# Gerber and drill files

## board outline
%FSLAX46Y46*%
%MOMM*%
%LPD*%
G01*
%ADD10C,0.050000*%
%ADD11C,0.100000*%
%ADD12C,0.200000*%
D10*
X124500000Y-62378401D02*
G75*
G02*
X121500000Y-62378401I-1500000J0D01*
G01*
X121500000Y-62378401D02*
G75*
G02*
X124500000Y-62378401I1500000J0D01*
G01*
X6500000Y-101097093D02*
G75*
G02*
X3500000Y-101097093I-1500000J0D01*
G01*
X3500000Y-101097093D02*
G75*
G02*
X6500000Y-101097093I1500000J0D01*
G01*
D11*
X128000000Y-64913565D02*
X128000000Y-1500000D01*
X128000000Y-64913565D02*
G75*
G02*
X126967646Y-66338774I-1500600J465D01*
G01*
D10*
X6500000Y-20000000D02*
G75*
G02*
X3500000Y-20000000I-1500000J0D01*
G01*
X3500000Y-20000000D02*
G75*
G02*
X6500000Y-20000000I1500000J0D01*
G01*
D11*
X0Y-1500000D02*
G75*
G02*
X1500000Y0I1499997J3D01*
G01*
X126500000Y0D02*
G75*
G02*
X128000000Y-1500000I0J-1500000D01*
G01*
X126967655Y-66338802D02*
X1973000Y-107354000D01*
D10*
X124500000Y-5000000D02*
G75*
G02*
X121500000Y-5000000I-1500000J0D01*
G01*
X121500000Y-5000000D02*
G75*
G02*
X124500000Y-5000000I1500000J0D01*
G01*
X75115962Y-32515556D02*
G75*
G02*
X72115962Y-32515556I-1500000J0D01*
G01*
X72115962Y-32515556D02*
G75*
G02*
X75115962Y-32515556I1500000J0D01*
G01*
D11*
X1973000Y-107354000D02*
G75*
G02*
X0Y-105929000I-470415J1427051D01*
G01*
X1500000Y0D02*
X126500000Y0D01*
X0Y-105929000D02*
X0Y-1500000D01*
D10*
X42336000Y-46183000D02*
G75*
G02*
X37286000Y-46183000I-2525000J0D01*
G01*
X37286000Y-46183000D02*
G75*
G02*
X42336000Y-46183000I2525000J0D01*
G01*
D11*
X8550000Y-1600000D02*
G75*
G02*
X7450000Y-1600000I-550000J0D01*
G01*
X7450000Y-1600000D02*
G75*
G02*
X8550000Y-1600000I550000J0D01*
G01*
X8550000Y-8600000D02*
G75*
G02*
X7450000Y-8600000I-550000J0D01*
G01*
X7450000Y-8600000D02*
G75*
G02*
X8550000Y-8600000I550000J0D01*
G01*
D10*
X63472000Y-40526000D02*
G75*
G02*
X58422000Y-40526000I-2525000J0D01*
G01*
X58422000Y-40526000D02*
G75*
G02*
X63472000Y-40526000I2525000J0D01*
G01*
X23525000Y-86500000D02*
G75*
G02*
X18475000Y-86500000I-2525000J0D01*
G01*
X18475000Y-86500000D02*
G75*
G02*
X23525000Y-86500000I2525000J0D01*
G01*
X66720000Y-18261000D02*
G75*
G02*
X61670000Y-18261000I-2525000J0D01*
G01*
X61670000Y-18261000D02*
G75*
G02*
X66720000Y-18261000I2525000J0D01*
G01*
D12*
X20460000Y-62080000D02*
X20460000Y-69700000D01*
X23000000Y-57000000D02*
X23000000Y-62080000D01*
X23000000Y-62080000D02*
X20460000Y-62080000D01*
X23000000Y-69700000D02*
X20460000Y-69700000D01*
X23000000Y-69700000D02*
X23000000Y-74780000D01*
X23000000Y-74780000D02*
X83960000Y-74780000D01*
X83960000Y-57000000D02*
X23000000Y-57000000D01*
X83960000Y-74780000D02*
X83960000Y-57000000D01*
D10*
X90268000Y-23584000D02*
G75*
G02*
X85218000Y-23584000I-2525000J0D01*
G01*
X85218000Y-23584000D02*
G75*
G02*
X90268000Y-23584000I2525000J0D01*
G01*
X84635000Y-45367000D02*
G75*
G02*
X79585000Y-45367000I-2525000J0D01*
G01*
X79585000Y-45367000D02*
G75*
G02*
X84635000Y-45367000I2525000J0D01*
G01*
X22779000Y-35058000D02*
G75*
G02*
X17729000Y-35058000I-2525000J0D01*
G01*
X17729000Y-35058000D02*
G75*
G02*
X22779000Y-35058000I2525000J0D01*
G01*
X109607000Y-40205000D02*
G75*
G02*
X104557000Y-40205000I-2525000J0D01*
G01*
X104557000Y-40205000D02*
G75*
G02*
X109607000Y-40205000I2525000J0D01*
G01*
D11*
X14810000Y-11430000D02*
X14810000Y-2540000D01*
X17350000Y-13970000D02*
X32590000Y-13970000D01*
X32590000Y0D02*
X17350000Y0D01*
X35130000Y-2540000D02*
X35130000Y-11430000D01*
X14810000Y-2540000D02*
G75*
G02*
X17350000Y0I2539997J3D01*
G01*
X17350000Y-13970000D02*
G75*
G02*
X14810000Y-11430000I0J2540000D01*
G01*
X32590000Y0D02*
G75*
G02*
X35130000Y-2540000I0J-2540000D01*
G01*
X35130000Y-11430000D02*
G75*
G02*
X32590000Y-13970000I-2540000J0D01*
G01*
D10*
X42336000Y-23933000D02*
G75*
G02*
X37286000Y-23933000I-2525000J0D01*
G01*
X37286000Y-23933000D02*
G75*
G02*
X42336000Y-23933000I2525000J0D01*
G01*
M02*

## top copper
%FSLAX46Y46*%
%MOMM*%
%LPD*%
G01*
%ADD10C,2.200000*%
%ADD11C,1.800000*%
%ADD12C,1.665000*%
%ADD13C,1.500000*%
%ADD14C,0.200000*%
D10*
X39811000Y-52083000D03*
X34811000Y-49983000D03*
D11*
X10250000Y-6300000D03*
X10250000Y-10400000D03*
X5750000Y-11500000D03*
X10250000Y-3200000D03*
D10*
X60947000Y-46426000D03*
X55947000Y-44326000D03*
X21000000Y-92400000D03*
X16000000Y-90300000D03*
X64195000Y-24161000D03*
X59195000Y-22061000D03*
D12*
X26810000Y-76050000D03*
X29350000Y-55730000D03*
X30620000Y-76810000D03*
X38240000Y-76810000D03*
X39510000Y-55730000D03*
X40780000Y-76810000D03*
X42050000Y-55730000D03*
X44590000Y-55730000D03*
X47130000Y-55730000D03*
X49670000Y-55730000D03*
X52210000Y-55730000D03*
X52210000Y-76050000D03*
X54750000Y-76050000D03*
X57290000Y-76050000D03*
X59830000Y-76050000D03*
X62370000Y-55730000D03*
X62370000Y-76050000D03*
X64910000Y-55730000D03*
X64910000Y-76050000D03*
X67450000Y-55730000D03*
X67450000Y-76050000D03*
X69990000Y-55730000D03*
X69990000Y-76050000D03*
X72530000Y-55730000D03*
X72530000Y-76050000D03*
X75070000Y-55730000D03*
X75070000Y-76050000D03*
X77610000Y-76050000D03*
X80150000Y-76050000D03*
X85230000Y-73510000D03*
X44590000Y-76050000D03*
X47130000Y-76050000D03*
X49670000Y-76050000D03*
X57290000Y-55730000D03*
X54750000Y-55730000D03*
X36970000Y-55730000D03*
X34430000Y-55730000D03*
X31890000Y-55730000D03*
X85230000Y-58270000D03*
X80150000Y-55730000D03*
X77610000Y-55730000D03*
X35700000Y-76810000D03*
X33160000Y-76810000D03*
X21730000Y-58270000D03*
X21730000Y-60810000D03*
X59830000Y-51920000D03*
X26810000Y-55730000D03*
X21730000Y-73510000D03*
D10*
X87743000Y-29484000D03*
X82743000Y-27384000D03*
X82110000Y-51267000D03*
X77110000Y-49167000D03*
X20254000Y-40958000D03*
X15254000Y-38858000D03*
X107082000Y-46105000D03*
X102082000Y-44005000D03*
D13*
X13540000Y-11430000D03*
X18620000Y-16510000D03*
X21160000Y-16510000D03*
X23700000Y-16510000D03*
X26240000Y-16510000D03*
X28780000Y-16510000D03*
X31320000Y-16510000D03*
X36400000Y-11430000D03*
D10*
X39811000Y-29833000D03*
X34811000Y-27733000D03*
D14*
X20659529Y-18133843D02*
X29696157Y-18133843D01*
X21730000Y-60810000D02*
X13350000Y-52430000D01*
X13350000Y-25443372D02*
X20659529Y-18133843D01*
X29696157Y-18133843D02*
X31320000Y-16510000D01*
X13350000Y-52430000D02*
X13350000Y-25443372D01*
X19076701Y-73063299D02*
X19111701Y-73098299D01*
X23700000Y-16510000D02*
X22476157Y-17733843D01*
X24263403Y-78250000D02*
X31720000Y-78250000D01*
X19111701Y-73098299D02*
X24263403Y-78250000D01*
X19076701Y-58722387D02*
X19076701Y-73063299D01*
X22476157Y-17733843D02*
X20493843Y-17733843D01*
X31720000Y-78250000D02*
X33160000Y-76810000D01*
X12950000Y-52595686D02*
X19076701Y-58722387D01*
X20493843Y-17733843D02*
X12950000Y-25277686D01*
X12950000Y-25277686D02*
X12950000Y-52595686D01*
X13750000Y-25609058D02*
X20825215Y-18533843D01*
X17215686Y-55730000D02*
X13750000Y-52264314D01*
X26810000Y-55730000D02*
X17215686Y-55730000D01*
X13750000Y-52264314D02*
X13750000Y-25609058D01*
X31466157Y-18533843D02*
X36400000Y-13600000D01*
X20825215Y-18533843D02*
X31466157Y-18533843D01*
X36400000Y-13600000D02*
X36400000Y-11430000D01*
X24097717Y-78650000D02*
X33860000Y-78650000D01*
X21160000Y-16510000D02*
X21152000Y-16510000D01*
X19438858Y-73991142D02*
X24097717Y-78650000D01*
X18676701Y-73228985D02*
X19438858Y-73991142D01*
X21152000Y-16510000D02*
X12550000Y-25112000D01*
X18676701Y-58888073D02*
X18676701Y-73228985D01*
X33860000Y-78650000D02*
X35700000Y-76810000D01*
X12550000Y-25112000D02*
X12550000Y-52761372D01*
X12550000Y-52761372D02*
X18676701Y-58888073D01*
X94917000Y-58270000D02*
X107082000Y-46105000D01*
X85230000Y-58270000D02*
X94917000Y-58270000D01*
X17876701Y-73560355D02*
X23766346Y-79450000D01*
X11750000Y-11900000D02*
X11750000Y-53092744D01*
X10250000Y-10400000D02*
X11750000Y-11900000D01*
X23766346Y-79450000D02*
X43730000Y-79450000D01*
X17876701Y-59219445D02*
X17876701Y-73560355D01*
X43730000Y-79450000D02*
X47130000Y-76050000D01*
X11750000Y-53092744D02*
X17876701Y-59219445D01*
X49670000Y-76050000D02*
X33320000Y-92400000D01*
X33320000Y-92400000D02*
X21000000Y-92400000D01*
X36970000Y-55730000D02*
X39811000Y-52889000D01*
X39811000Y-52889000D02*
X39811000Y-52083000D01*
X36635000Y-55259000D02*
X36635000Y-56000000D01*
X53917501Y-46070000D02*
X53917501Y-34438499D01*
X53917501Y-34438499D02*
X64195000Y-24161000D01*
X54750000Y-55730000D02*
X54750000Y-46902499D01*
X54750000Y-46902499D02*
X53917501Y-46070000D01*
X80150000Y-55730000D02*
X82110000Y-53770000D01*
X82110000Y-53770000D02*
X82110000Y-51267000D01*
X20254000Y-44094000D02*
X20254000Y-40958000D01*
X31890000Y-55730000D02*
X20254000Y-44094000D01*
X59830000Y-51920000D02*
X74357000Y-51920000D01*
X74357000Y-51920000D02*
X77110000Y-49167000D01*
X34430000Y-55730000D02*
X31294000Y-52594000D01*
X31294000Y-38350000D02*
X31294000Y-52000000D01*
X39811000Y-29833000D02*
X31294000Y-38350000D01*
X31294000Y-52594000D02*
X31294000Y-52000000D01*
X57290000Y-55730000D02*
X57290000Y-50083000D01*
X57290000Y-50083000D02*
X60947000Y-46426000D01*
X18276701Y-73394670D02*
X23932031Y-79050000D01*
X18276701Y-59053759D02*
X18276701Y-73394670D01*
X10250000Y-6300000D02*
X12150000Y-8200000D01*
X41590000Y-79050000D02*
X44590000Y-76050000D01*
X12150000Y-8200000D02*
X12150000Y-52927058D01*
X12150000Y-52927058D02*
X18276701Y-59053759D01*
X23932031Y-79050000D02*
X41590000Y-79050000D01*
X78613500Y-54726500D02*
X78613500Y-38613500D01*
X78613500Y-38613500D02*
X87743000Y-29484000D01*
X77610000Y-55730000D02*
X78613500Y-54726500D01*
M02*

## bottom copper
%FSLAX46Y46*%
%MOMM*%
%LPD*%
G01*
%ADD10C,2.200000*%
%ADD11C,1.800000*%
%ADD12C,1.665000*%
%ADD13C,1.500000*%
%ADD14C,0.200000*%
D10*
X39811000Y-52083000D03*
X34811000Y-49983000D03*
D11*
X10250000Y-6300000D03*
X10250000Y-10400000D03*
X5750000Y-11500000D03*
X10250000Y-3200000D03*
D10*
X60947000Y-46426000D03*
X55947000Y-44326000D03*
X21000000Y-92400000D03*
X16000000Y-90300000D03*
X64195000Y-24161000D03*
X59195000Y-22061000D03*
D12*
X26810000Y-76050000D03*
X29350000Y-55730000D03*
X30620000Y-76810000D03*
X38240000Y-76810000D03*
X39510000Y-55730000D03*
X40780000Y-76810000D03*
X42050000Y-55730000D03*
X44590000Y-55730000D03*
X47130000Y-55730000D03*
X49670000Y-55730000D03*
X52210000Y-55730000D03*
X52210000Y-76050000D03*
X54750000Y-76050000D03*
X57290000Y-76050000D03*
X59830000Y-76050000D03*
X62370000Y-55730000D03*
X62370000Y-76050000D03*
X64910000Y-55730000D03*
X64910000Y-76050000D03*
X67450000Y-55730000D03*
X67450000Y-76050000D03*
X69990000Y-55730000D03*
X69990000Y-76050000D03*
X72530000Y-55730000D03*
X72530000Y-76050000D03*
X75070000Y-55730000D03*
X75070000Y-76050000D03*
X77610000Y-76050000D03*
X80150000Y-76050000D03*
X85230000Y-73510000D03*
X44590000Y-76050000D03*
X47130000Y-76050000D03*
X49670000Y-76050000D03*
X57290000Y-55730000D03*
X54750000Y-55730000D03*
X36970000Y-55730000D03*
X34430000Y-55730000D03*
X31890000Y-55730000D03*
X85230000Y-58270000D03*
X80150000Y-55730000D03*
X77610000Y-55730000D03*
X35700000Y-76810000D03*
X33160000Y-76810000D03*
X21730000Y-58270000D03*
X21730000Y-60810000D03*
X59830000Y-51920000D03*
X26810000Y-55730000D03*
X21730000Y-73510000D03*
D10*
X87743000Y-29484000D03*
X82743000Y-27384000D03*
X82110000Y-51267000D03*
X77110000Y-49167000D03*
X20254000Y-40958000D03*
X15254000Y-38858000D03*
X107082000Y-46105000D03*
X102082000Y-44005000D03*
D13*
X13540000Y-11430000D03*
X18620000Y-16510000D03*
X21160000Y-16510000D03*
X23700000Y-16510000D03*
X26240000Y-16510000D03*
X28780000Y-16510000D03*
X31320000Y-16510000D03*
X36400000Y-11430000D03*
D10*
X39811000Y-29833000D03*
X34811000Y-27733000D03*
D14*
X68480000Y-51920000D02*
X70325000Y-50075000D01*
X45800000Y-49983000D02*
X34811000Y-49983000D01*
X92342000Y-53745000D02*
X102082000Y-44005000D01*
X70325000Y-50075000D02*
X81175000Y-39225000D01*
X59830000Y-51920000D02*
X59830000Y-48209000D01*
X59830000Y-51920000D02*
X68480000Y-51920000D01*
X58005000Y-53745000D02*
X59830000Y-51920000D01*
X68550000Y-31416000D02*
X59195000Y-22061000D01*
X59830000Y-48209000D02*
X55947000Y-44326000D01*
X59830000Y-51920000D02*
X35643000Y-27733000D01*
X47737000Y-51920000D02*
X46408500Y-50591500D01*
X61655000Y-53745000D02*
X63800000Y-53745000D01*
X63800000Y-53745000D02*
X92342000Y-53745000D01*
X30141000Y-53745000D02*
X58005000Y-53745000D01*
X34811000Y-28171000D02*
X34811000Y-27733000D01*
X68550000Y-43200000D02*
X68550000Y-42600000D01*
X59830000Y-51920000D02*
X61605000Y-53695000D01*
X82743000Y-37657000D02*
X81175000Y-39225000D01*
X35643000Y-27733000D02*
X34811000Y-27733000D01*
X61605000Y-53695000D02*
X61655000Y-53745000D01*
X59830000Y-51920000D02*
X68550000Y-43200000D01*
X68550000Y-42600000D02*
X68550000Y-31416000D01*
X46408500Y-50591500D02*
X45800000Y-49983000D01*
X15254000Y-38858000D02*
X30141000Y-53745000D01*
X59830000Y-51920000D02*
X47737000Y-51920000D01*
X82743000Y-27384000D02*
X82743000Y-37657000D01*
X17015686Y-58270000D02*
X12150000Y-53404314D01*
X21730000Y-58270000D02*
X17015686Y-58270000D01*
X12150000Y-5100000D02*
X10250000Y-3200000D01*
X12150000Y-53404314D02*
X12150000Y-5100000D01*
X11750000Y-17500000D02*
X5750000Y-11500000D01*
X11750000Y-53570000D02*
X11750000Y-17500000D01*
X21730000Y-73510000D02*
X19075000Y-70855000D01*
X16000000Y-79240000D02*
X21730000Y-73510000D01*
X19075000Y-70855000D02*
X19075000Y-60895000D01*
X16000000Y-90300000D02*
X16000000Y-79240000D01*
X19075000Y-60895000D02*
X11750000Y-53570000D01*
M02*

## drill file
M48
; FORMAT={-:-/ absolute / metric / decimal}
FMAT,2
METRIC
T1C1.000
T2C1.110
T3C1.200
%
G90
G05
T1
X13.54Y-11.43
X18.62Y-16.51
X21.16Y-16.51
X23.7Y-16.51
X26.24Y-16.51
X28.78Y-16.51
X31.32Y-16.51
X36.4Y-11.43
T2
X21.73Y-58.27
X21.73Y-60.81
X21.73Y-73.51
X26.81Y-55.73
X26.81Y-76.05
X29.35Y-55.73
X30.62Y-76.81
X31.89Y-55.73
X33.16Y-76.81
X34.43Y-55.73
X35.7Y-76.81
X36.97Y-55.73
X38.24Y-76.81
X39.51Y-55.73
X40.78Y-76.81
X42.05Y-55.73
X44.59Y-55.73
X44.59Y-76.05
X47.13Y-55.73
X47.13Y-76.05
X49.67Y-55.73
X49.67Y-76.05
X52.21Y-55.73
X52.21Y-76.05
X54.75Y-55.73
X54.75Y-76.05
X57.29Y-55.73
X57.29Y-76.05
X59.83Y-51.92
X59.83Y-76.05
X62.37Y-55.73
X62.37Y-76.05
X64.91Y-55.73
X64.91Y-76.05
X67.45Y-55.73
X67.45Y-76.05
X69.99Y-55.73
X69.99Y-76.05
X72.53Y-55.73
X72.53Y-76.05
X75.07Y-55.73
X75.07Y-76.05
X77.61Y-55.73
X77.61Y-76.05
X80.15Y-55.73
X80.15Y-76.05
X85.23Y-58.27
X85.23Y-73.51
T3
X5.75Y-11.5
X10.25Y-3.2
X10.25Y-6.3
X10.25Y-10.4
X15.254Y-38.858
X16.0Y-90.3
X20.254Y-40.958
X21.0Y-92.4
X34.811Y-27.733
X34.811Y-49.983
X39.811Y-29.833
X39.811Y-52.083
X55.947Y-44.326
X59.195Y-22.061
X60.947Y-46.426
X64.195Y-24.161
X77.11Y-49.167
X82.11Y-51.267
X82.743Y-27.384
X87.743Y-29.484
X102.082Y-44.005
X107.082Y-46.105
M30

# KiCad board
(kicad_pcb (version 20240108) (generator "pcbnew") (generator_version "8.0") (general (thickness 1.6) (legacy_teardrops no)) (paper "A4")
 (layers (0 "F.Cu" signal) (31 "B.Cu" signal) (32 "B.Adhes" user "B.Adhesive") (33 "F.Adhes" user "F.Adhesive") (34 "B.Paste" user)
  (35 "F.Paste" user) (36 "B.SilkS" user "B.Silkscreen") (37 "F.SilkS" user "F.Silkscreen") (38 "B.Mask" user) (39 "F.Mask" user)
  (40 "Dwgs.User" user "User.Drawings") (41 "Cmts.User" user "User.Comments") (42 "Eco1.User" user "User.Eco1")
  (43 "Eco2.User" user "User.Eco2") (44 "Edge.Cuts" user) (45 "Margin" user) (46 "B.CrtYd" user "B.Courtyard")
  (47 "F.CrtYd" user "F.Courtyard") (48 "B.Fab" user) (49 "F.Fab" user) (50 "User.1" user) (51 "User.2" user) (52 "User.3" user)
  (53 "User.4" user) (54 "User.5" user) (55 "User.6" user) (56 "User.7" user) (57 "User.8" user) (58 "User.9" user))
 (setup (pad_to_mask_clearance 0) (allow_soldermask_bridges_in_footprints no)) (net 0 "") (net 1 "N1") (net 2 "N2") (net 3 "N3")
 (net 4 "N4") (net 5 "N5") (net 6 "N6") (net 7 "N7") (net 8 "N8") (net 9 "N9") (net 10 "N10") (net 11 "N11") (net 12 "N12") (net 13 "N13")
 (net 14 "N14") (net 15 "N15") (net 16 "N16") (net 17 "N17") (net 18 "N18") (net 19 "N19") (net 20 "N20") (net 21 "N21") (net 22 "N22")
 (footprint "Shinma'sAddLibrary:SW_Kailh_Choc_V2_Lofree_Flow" (layer "F.Cu") (at 39.811 46.183)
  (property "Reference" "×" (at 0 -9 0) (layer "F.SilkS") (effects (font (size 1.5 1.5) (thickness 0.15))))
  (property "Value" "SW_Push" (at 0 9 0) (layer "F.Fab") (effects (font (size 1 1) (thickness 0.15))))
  (fp_circle (center 0 0) (end 2.525 0) (stroke (width 0.05) (type default)) (fill none) (layer "Edge.Cuts"))
  (pad "1" thru_hole circle (at 0 5.9) (size 2.2 2.2) (drill 1.2) (layers "*.Cu" "*.Mask") (remove_unused_layers no) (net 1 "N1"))
  (pad "2" thru_hole circle (at -5 3.8) (size 2.2 2.2) (drill 1.2) (layers "*.Cu" "*.Mask") (remove_unused_layers no) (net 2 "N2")))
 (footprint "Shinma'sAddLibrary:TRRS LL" (layer "F.Cu") (at 5 12 90)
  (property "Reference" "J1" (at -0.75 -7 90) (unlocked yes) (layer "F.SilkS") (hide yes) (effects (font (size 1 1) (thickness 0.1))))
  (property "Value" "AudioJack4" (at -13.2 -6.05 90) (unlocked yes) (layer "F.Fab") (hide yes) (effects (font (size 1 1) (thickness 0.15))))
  (fp_circle (center 10.4 3) (end 10.95 3) (stroke (width 0.1) (type default)) (fill none) (layer "Edge.Cuts"))
  (fp_circle (center 3.4 3) (end 3.95 3) (stroke (width 0.1) (type default)) (fill none) (layer "Edge.Cuts"))
  (pad "R1" thru_hole circle (at 5.7 5.25 90) (size 1.8 1.8) (drill 1.2) (layers "*.Cu" "*.Mask") (remove_unused_layers no) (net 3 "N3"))
  (pad "R2" thru_hole circle (at 1.6 5.25 90) (size 1.8 1.8) (drill 1.2) (layers "*.Cu" "*.Mask") (remove_unused_layers no) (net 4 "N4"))
  (pad "S" thru_hole circle (at 0.5 0.75 90) (size 1.8 1.8) (drill 1.2) (layers "*.Cu" "*.Mask") (remove_unused_layers no) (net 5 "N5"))
  (pad "T" thru_hole circle (at 8.8 5.25 90) (size 1.8 1.8) (drill 1.2) (layers "*.Cu" "*.Mask") (remove_unused_layers no) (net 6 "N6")))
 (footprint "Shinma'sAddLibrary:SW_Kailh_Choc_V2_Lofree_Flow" (layer "F.Cu") (at 60.947 40.526)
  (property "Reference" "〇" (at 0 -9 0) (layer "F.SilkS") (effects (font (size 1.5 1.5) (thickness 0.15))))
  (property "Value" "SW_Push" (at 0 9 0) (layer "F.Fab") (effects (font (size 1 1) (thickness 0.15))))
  (fp_circle (center 0 0) (end 2.525 0) (stroke (width 0.05) (type default)) (fill none) (layer "Edge.Cuts"))
  (pad "1" thru_hole circle (at 0 5.9) (size 2.2 2.2) (drill 1.2) (layers "*.Cu" "*.Mask") (remove_unused_layers no) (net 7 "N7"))
  (pad "2" thru_hole circle (at -5 3.8) (size 2.2 2.2) (drill 1.2) (layers "*.Cu" "*.Mask") (remove_unused_layers no) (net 2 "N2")))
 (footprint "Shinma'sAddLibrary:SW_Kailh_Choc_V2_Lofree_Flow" (layer "F.Cu") (at 21 86.5)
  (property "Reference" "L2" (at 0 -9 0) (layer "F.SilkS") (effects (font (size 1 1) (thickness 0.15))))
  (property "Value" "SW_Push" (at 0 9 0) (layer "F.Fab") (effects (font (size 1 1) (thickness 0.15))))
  (fp_circle (center 0 0) (end 2.525 0) (stroke (width 0.05) (type default)) (fill none) (layer "Edge.Cuts"))
  (pad "1" thru_hole circle (at 0 5.9) (size 2.2 2.2) (drill 1.2) (layers "*.Cu" "*.Mask") (remove_unused_layers no) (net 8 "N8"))
  (pad "2" thru_hole circle (at -5 3.8) (size 2.2 2.2) (drill 1.2) (layers "*.Cu" "*.Mask") (remove_unused_layers no) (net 5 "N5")))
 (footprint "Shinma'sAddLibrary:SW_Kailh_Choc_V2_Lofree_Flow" (layer "F.Cu") (at 64.195 18.261)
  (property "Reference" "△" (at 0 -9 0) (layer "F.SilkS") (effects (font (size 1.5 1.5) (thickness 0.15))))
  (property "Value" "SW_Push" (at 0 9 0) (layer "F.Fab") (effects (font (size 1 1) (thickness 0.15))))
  (fp_circle (center 0 0) (end 2.525 0) (stroke (width 0.05) (type default)) (fill none) (layer "Edge.Cuts"))
  (pad "1" thru_hole circle (at 0 5.9) (size 2.2 2.2) (drill 1.2) (layers "*.Cu" "*.Mask") (remove_unused_layers no) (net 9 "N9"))
  (pad "2" thru_hole circle (at -5 3.8) (size 2.2 2.2) (drill 1.2) (layers "*.Cu" "*.Mask") (remove_unused_layers no) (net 2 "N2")))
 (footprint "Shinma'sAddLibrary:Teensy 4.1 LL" (layer "F.Cu") (at 24.27 58.27)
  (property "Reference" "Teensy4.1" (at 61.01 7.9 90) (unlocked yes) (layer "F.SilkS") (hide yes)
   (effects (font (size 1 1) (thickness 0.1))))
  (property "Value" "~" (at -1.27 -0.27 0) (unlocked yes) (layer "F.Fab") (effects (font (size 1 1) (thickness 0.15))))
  (fp_line (start -3.81 3.81) (end -3.81 11.43) (stroke (width 0.2) (type default)) (layer "Edge.Cuts"))
  (fp_line (start -1.27 -1.27) (end -1.27 3.81) (stroke (width 0.2) (type default)) (layer "Edge.Cuts"))
  (fp_line (start -1.27 3.81) (end -3.81 3.81) (stroke (width 0.2) (type default)) (layer "Edge.Cuts"))
  (fp_line (start -1.27 11.43) (end -3.81 11.43) (stroke (width 0.2) (type default)) (layer "Edge.Cuts"))
  (fp_line (start -1.27 11.43) (end -1.27 16.51) (stroke (width 0.2) (type default)) (layer "Edge.Cuts"))
  (fp_line (start -1.27 16.51) (end 59.69 16.51) (stroke (width 0.2) (type solid)) (layer "Edge.Cuts"))
  (fp_line (start 59.69 -1.27) (end -1.27 -1.27) (stroke (width 0.2) (type solid)) (layer "Edge.Cuts"))
  (fp_line (start 59.69 16.51) (end 59.69 -1.27) (stroke (width 0.2) (type solid)) (layer "Edge.Cuts"))
  (pad "" thru_hole circle (at 2.54 17.78) (size 1.665 1.665) (drill 1.11) (layers "*.Cu" "*.Mask") (remove_unused_layers no))
  (pad "" thru_hole circle (at 5.08 -2.54) (size 1.665 1.665) (drill 1.11) (layers "*.Cu" "*.Mask") (remove_unused_layers no))
  (pad "" thru_hole circle (at 6.35 18.54) (size 1.665 1.665) (drill 1.11) (layers "*.Cu" "*.Mask") (remove_unused_layers no))
  (pad "" thru_hole circle (at 13.97 18.54) (size 1.665 1.665) (drill 1.11) (layers "*.Cu" "*.Mask") (remove_unused_layers no))
  (pad "" thru_hole circle (at 15.24 -2.54) (size 1.665 1.665) (drill 1.11) (layers "*.Cu" "*.Mask") (remove_unused_layers no))
  (pad "" thru_hole circle (at 16.51 18.54) (size 1.665 1.665) (drill 1.11) (layers "*.Cu" "*.Mask") (remove_unused_layers no))
  (pad "" thru_hole circle (at 17.78 -2.54) (size 1.665 1.665) (drill 1.11) (layers "*.Cu" "*.Mask") (remove_unused_layers no))
  (pad "" thru_hole circle (at 20.32 -2.54) (size 1.665 1.665) (drill 1.11) (layers "*.Cu" "*.Mask") (remove_unused_layers no))
  (pad "" thru_hole circle (at 22.86 -2.54) (size 1.665 1.665) (drill 1.11) (layers "*.Cu" "*.Mask") (remove_unused_layers no))
  (pad "" thru_hole circle (at 25.4 -2.54) (size 1.665 1.665) (drill 1.11) (layers "*.Cu" "*.Mask") (remove_unused_layers no))
  (pad "" thru_hole circle (at 27.94 -2.54) (size 1.665 1.665) (drill 1.11) (layers "*.Cu" "*.Mask") (remove_unused_layers no))
  (pad "" thru_hole circle (at 27.94 17.78) (size 1.665 1.665) (drill 1.11) (layers "*.Cu" "*.Mask") (remove_unused_layers no))
  (pad "" thru_hole circle (at 30.48 17.78) (size 1.665 1.665) (drill 1.11) (layers "*.Cu" "*.Mask") (remove_unused_layers no))
  (pad "" thru_hole circle (at 33.02 17.78) (size 1.665 1.665) (drill 1.11) (layers "*.Cu" "*.Mask") (remove_unused_layers no))
  (pad "" thru_hole circle (at 35.56 17.78) (size 1.665 1.665) (drill 1.11) (layers "*.Cu" "*.Mask") (remove_unused_layers no))
  (pad "" thru_hole circle (at 38.1 -2.54) (size 1.665 1.665) (drill 1.11) (layers "*.Cu" "*.Mask") (remove_unused_layers no))
  (pad "" thru_hole circle (at 38.1 17.78) (size 1.665 1.665) (drill 1.11) (layers "*.Cu" "*.Mask") (remove_unused_layers no))
  (pad "" thru_hole circle (at 40.64 -2.54) (size 1.665 1.665) (drill 1.11) (layers "*.Cu" "*.Mask") (remove_unused_layers no))
  (pad "" thru_hole circle (at 40.64 17.78) (size 1.665 1.665) (drill 1.11) (layers "*.Cu" "*.Mask") (remove_unused_layers no))
  (pad "" thru_hole circle (at 43.18 -2.54) (size 1.665 1.665) (drill 1.11) (layers "*.Cu" "*.Mask") (remove_unused_layers no))
  (pad "" thru_hole circle (at 43.18 17.78) (size 1.665 1.665) (drill 1.11) (layers "*.Cu" "*.Mask") (remove_unused_layers no))
  (pad "" thru_hole circle (at 45.72 -2.54) (size 1.665 1.665) (drill 1.11) (layers "*.Cu" "*.Mask") (remove_unused_layers no))
  (pad "" thru_hole circle (at 45.72 17.78) (size 1.665 1.665) (drill 1.11) (layers "*.Cu" "*.Mask") (remove_unused_layers no))
  (pad "" thru_hole circle (at 48.26 -2.54) (size 1.665 1.665) (drill 1.11) (layers "*.Cu" "*.Mask") (remove_unused_layers no))
  (pad "" thru_hole circle (at 48.26 17.78) (size 1.665 1.665) (drill 1.11) (layers "*.Cu" "*.Mask") (remove_unused_layers no))
  (pad "" thru_hole circle (at 50.8 -2.54) (size 1.665 1.665) (drill 1.11) (layers "*.Cu" "*.Mask") (remove_unused_layers no))
  (pad "" thru_hole circle (at 50.8 17.78) (size 1.665 1.665) (drill 1.11) (layers "*.Cu" "*.Mask") (remove_unused_layers no))
  (pad "" thru_hole circle (at 53.34 17.78) (size 1.665 1.665) (drill 1.11) (layers "*.Cu" "*.Mask") (remove_unused_layers no))
  (pad "" thru_hole circle (at 55.88 17.78) (size 1.665 1.665) (drill 1.11) (layers "*.Cu" "*.Mask") (remove_unused_layers no))
  (pad "" thru_hole circle (at 60.96 15.24) (size 1.665 1.665) (drill 1.11) (layers "*.Cu" "*.Mask") (remove_unused_layers no))
  (pad "7" thru_hole circle (at 20.32 17.78) (size 1.665 1.665) (drill 1.11) (layers "*.Cu" "*.Mask") (remove_unused_layers no) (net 3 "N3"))
  (pad "8" thru_hole circle (at 22.86 17.78) (size 1.665 1.665) (drill 1.11) (layers "*.Cu" "*.Mask") (remove_unused_layers no) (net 4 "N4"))
  (pad "9" thru_hole circle (at 25.4 17.78) (size 1.665 1.665) (drill 1.11) (layers "*.Cu" "*.Mask") (remove_unused_layers no) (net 8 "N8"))
  (pad "13" thru_hole circle (at 33.02 -2.54) (size 1.665 1.665) (drill 1.11) (layers "*.Cu" "*.Mask") (remove_unused_layers no)
   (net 7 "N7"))
  (pad "14" thru_hole circle (at 30.48 -2.54) (size 1.665 1.665) (drill 1.11) (layers "*.Cu" "*.Mask") (remove_unused_layers no)
   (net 9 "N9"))
  (pad "21" thru_hole circle (at 12.7 -2.54) (size 1.665 1.665) (drill 1.11) (layers "*.Cu" "*.Mask") (remove_unused_layers no) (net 1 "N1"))
  (pad "22" thru_hole circle (at 10.16 -2.54) (size 1.665 1.665) (drill 1.11) (layers "*.Cu" "*.Mask") (remove_unused_layers no)
   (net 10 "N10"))
  (pad "23" thru_hole circle (at 7.62 -2.54) (size 1.665 1.665) (drill 1.11) (layers "*.Cu" "*.Mask") (remove_unused_layers no)
   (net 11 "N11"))
  (pad "33" thru_hole circle (at 60.96 0) (size 1.665 1.665) (drill 1.11) (layers "*.Cu" "*.Mask") (remove_unused_layers no) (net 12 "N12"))
  (pad "34" thru_hole circle (at 55.88 -2.54) (size 1.665 1.665) (drill 1.11) (layers "*.Cu" "*.Mask") (remove_unused_layers no)
   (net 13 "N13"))
  (pad "35" thru_hole circle (at 53.34 -2.54) (size 1.665 1.665) (drill 1.11) (layers "*.Cu" "*.Mask") (remove_unused_layers no)
   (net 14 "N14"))
  (pad "50" thru_hole circle (at 11.43 18.54) (size 1.665 1.665) (drill 1.11) (layers "*.Cu" "*.Mask") (remove_unused_layers no)
   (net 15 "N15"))
  (pad "51" thru_hole circle (at 8.89 18.54) (size 1.665 1.665) (drill 1.11) (layers "*.Cu" "*.Mask") (remove_unused_layers no)
   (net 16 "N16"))
  (pad "55" thru_hole circle (at -2.54 0) (size 1.665 1.665) (drill 1.11) (layers "*.Cu" "*.Mask") (remove_unused_layers no) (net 6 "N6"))
  (pad "68" thru_hole circle (at -2.54 2.54) (size 1.665 1.665) (drill 1.11) (layers "*.Cu" "*.Mask") (remove_unused_layers no)
   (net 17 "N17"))
  (pad "69" thru_hole circle (at 35.56 -6.35) (size 1.665 1.665) (drill 1.11) (layers "*.Cu" "*.Mask") (remove_unused_layers no)
   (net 2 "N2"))
  (pad "70" thru_hole circle (at 2.54 -2.54) (size 1.665 1.665) (drill 1.11) (layers "*.Cu" "*.Mask") (remove_unused_layers no)
   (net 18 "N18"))
  (pad "71" thru_hole circle (at -2.54 15.24) (size 1.665 1.665) (drill 1.11) (layers "*.Cu" "*.Mask") (remove_unused_layers no)
   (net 5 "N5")))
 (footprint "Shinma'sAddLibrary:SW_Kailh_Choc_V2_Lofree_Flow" (layer "F.Cu") (at 87.743 23.584)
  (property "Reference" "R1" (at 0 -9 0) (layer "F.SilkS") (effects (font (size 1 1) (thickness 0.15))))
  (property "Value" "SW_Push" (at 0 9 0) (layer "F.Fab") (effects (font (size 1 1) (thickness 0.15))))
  (fp_circle (center 0 0) (end 2.525 0) (stroke (width 0.05) (type default)) (fill none) (layer "Edge.Cuts"))
  (pad "1" thru_hole circle (at 0 5.9) (size 2.2 2.2) (drill 1.2) (layers "*.Cu" "*.Mask") (remove_unused_layers no) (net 14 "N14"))
  (pad "2" thru_hole circle (at -5 3.8) (size 2.2 2.2) (drill 1.2) (layers "*.Cu" "*.Mask") (remove_unused_layers no) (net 2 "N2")))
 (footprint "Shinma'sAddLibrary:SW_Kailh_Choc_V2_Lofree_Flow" (layer "F.Cu") (at 82.11 45.367)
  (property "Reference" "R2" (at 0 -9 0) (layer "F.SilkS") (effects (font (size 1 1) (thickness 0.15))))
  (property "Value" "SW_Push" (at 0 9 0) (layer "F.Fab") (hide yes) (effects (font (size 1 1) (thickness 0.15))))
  (fp_circle (center 0 0) (end 2.525 0) (stroke (width 0.05) (type default)) (fill none) (layer "Edge.Cuts"))
  (pad "1" thru_hole circle (at 0 5.9) (size 2.2 2.2) (drill 1.2) (layers "*.Cu" "*.Mask") (remove_unused_layers no) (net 13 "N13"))
  (pad "2" thru_hole circle (at -5 3.8) (size 2.2 2.2) (drill 1.2) (layers "*.Cu" "*.Mask") (remove_unused_layers no) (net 2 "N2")))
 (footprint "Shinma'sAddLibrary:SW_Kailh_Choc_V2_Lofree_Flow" (layer "F.Cu") (at 20.254 35.058)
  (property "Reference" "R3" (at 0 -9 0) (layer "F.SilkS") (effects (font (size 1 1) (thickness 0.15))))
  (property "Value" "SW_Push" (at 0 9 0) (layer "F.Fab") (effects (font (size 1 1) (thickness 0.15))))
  (fp_circle (center 0 0) (end 2.525 0) (stroke (width 0.05) (type default)) (fill none) (layer "Edge.Cuts"))
  (pad "1" thru_hole circle (at 0 5.9) (size 2.2 2.2) (drill 1.2) (layers "*.Cu" "*.Mask") (remove_unused_layers no) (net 11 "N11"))
  (pad "2" thru_hole circle (at -5 3.8) (size 2.2 2.2) (drill 1.2) (layers "*.Cu" "*.Mask") (remove_unused_layers no) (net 2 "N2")))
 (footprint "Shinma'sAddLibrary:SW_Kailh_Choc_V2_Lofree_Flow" (layer "F.Cu") (at 107.082 40.205)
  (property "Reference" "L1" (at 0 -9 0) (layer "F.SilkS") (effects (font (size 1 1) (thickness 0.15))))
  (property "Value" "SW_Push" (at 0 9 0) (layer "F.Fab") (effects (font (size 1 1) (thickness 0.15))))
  (fp_circle (center 0 0) (end 2.525 0) (stroke (width 0.05) (type default)) (fill none) (layer "Edge.Cuts"))
  (pad "1" thru_hole circle (at 0 5.9) (size 2.2 2.2) (drill 1.2) (layers "*.Cu" "*.Mask") (remove_unused_layers no) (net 12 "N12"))
  (pad "2" thru_hole circle (at -5 3.8) (size 2.2 2.2) (drill 1.2) (layers "*.Cu" "*.Mask") (remove_unused_layers no) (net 2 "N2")))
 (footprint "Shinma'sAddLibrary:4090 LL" (layer "F.Cu") (at 14.81 0)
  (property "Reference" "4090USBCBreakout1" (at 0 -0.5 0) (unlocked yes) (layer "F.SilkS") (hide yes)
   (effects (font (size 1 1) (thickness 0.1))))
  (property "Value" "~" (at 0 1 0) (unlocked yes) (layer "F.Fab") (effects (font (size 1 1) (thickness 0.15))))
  (fp_line (start 0 11.43) (end 0 2.54) (stroke (width 0.1) (type default)) (layer "Edge.Cuts"))
  (fp_line (start 2.54 13.97) (end 17.78 13.97) (stroke (width 0.1) (type default)) (layer "Edge.Cuts"))
  (fp_line (start 17.78 0) (end 2.54 0) (stroke (width 0.1) (type default)) (layer "Edge.Cuts"))
  (fp_line (start 20.32 2.54) (end 20.32 11.43) (stroke (width 0.1) (type default)) (layer "Edge.Cuts"))
  (fp_arc (start 0 2.54) (mid 0.743948 0.743948) (end 2.54 0) (stroke (width 0.1) (type default)) (layer "Edge.Cuts"))
  (fp_arc (start 2.54 13.97) (mid 0.743949 13.226051) (end 0 11.43) (stroke (width 0.1) (type default)) (layer "Edge.Cuts"))
  (fp_arc (start 17.78 0) (mid 19.576051 0.743949) (end 20.32 2.54) (stroke (width 0.1) (type default)) (layer "Edge.Cuts"))
  (fp_arc (start 20.32 11.43) (mid 19.576051 13.226051) (end 17.78 13.97) (stroke (width 0.1) (type default)) (layer "Edge.Cuts"))
  (pad "1" thru_hole circle (at -1.27 11.43) (size 1.5 1.5) (drill 1) (layers "*.Cu" "*.Mask") (remove_unused_layers no) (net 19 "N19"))
  (pad "2" thru_hole circle (at 3.81 16.51) (size 1.5 1.5) (drill 1) (layers "*.Cu" "*.Mask") (remove_unused_layers no) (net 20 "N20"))
  (pad "3" thru_hole circle (at 6.35 16.51) (size 1.5 1.5) (drill 1) (layers "*.Cu" "*.Mask") (remove_unused_layers no) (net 15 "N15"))
  (pad "4" thru_hole circle (at 8.89 16.51) (size 1.5 1.5) (drill 1) (layers "*.Cu" "*.Mask") (remove_unused_layers no) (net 16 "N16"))
  (pad "5" thru_hole circle (at 11.43 16.51) (size 1.5 1.5) (drill 1) (layers "*.Cu" "*.Mask") (remove_unused_layers no) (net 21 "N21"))
  (pad "6" thru_hole circle (at 13.97 16.51) (size 1.5 1.5) (drill 1) (layers "*.Cu" "*.Mask") (remove_unused_layers no) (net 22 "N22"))
  (pad "7" thru_hole circle (at 16.51 16.51) (size 1.5 1.5) (drill 1) (layers "*.Cu" "*.Mask") (remove_unused_layers no) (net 17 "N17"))
  (pad "8" thru_hole circle (at 21.59 11.43) (size 1.5 1.5) (drill 1) (layers "*.Cu" "*.Mask") (remove_unused_layers no) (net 18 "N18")))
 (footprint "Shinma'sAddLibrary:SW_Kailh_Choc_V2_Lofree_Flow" (layer "F.Cu") (at 39.811 23.933)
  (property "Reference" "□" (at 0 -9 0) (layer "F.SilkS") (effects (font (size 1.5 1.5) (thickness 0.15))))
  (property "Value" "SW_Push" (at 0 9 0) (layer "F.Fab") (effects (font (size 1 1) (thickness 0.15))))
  (fp_circle (center 0 0) (end 2.525 0) (stroke (width 0.05) (type default)) (fill none) (layer "Edge.Cuts"))
  (pad "1" thru_hole circle (at 0 5.9) (size 2.2 2.2) (drill 1.2) (layers "*.Cu" "*.Mask") (remove_unused_layers no) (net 10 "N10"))
  (pad "2" thru_hole circle (at -5 3.8) (size 2.2 2.2) (drill 1.2) (layers "*.Cu" "*.Mask") (remove_unused_layers no) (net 2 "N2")))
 (gr_circle (center 123 62.378401) (end 124.5 62.378401) (stroke (width 0.05) (type default)) (fill none) (layer "Edge.Cuts"))
 (gr_circle (center 5 101.097093) (end 6.5 101.097093) (stroke (width 0.05) (type default)) (fill none) (layer "Edge.Cuts"))
 (gr_line (start 128 64.913565) (end 128 1.5) (stroke (width 0.1) (type default)) (layer "Edge.Cuts"))
 (gr_arc (start 128 64.913565) (mid 127.714684 65.7934) (end 126.967655 66.338802) (stroke (width 0.1) (type default)) (layer "Edge.Cuts"))
 (gr_circle (center 5 20) (end 6.5 20) (stroke (width 0.05) (type default)) (fill none) (layer "Edge.Cuts"))
 (gr_arc (start 0 1.5) (mid 0.439339 0.439339) (end 1.5 0) (stroke (width 0.1) (type default)) (layer "Edge.Cuts"))
 (gr_arc (start 126.5 0) (mid 127.56066 0.43934) (end 128 1.5) (stroke (width 0.1) (type default)) (layer "Edge.Cuts"))
 (gr_line (start 126.967655 66.338802) (end 1.973 107.354) (stroke (width 0.1) (type default)) (layer "Edge.Cuts"))
 (gr_circle (center 123 5) (end 124.5 5) (stroke (width 0.05) (type default)) (fill none) (layer "Edge.Cuts"))
 (gr_circle (center 73.615962 32.515556) (end 75.115962 32.515556) (stroke (width 0.05) (type default)) (fill none) (layer "Edge.Cuts"))
 (gr_arc (start 1.973 107.354) (mid 0.622812 107.145048) (end 0 105.929) (stroke (width 0.1) (type default)) (layer "Edge.Cuts"))
 (gr_line (start 1.5 0) (end 126.5 0) (stroke (width 0.1) (type default)) (layer "Edge.Cuts"))
 (gr_line (start 0 105.929) (end 0 1.5) (stroke (width 0.1) (type default)) (layer "Edge.Cuts"))
 (segment (start 20.659529 18.133843) (end 29.696157 18.133843) (width 0.2) (layer "F.Cu") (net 17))
 (segment (start 21.73 60.81) (end 13.35 52.43) (width 0.2) (layer "F.Cu") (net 17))
 (segment (start 13.35 25.443372) (end 20.659529 18.133843) (width 0.2) (layer "F.Cu") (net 17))
 (segment (start 29.696157 18.133843) (end 31.32 16.51) (width 0.2) (layer "F.Cu") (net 17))
 (segment (start 13.35 52.43) (end 13.35 25.443372) (width 0.2) (layer "F.Cu") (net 17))
 (segment (start 19.076701 73.063299) (end 19.111701 73.098299) (width 0.2) (layer "F.Cu") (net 16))
 (segment (start 23.7 16.51) (end 22.476157 17.733843) (width 0.2) (layer "F.Cu") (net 16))
 (segment (start 24.263403 78.25) (end 31.72 78.25) (width 0.2) (layer "F.Cu") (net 16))
 (segment (start 19.111701 73.098299) (end 24.263403 78.25) (width 0.2) (layer "F.Cu") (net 16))
 (segment (start 19.076701 58.722387) (end 19.076701 73.063299) (width 0.2) (layer "F.Cu") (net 16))
 (segment (start 22.476157 17.733843) (end 20.493843 17.733843) (width 0.2) (layer "F.Cu") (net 16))
 (segment (start 31.72 78.25) (end 33.16 76.81) (width 0.2) (layer "F.Cu") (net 16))
 (segment (start 12.95 52.595686) (end 19.076701 58.722387) (width 0.2) (layer "F.Cu") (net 16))
 (segment (start 20.493843 17.733843) (end 12.95 25.277686) (width 0.2) (layer "F.Cu") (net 16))
 (segment (start 12.95 25.277686) (end 12.95 52.595686) (width 0.2) (layer "F.Cu") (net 16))
 (segment (start 13.75 25.609058) (end 20.825215 18.533843) (width 0.2) (layer "F.Cu") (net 18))
 (segment (start 17.215686 55.73) (end 13.75 52.264314) (width 0.2) (layer "F.Cu") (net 18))
 (segment (start 26.81 55.73) (end 17.215686 55.73) (width 0.2) (layer "F.Cu") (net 18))
 (segment (start 13.75 52.264314) (end 13.75 25.609058) (width 0.2) (layer "F.Cu") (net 18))
 (segment (start 31.466157 18.533843) (end 36.4 13.6) (width 0.2) (layer "F.Cu") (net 18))
 (segment (start 20.825215 18.533843) (end 31.466157 18.533843) (width 0.2) (layer "F.Cu") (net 18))
 (segment (start 36.4 13.6) (end 36.4 11.43) (width 0.2) (layer "F.Cu") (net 18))
 (segment (start 24.097717 78.65) (end 33.86 78.65) (width 0.2) (layer "F.Cu") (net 15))
 (segment (start 21.16 16.51) (end 21.152 16.51) (width 0.2) (layer "F.Cu") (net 15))
 (segment (start 19.438858 73.991142) (end 24.097717 78.65) (width 0.2) (layer "F.Cu") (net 15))
 (segment (start 18.676701 73.228985) (end 19.438858 73.991142) (width 0.2) (layer "F.Cu") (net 15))
 (segment (start 21.152 16.51) (end 12.55 25.112) (width 0.2) (layer "F.Cu") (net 15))
 (segment (start 18.676701 58.888073) (end 18.676701 73.228985) (width 0.2) (layer "F.Cu") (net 15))
 (segment (start 33.86 78.65) (end 35.7 76.81) (width 0.2) (layer "F.Cu") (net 15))
 (segment (start 12.55 25.112) (end 12.55 52.761372) (width 0.2) (layer "F.Cu") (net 15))
 (segment (start 12.55 52.761372) (end 18.676701 58.888073) (width 0.2) (layer "F.Cu") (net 15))
 (segment (start 94.917 58.27) (end 107.082 46.105) (width 0.2) (layer "F.Cu") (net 12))
 (segment (start 85.23 58.27) (end 94.917 58.27) (width 0.2) (layer "F.Cu") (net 12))
 (segment (start 17.876701 73.560355) (end 23.766346 79.45) (width 0.2) (layer "F.Cu") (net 4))
 (segment (start 11.75 11.9) (end 11.75 53.092744) (width 0.2) (layer "F.Cu") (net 4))
 (segment (start 10.25 10.4) (end 11.75 11.9) (width 0.2) (layer "F.Cu") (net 4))
 (segment (start 23.766346 79.45) (end 43.73 79.45) (width 0.2) (layer "F.Cu") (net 4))
 (segment (start 17.876701 59.219445) (end 17.876701 73.560355) (width 0.2) (layer "F.Cu") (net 4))
 (segment (start 43.73 79.45) (end 47.13 76.05) (width 0.2) (layer "F.Cu") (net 4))
 (segment (start 11.75 53.092744) (end 17.876701 59.219445) (width 0.2) (layer "F.Cu") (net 4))
 (segment (start 49.67 76.05) (end 33.32 92.4) (width 0.2) (layer "F.Cu") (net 8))
 (segment (start 33.32 92.4) (end 21 92.4) (width 0.2) (layer "F.Cu") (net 8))
 (segment (start 36.97 55.73) (end 39.811 52.889) (width 0.2) (layer "F.Cu") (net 1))
 (segment (start 39.811 52.889) (end 39.811 52.083) (width 0.2) (layer "F.Cu") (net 1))
 (segment (start 36.635 55.259) (end 36.635 56) (width 0.2) (layer "F.Cu") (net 1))
 (segment (start 53.917501 46.07) (end 53.917501 34.438499) (width 0.2) (layer "F.Cu") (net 9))
 (segment (start 53.917501 34.438499) (end 64.195 24.161) (width 0.2) (layer "F.Cu") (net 9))
 (segment (start 54.75 55.73) (end 54.75 46.902499) (width 0.2) (layer "F.Cu") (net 9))
 (segment (start 54.75 46.902499) (end 53.917501 46.07) (width 0.2) (layer "F.Cu") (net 9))
 (segment (start 80.15 55.73) (end 82.11 53.77) (width 0.2) (layer "F.Cu") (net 13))
 (segment (start 82.11 53.77) (end 82.11 51.267) (width 0.2) (layer "F.Cu") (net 13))
 (segment (start 20.254 44.094) (end 20.254 40.958) (width 0.2) (layer "F.Cu") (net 11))
 (segment (start 31.89 55.73) (end 20.254 44.094) (width 0.2) (layer "F.Cu") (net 11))
 (segment (start 59.83 51.92) (end 74.357 51.92) (width 0.2) (layer "F.Cu") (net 2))
 (segment (start 74.357 51.92) (end 77.11 49.167) (width 0.2) (layer "F.Cu") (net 2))
 (segment (start 68.48 51.92) (end 70.325 50.075) (width 0.2) (layer "B.Cu") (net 2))
 (segment (start 45.8 49.983) (end 34.811 49.983) (width 0.2) (layer "B.Cu") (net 2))
 (segment (start 92.342 53.745) (end 102.082 44.005) (width 0.2) (layer "B.Cu") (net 2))
 (segment (start 70.325 50.075) (end 81.175 39.225) (width 0.2) (layer "B.Cu") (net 2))
 (segment (start 59.83 51.92) (end 59.83 48.209) (width 0.2) (layer "B.Cu") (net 2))
 (segment (start 59.83 51.92) (end 68.48 51.92) (width 0.2) (layer "B.Cu") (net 2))
 (segment (start 58.005 53.745) (end 59.83 51.92) (width 0.2) (layer "B.Cu") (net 2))
 (segment (start 68.55 31.416) (end 59.195 22.061) (width 0.2) (layer "B.Cu") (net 2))
 (segment (start 59.83 48.209) (end 55.947 44.326) (width 0.2) (layer "B.Cu") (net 2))
 (segment (start 59.83 51.92) (end 35.643 27.733) (width 0.2) (layer "B.Cu") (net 2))
 (segment (start 47.737 51.92) (end 46.4085 50.5915) (width 0.2) (layer "B.Cu") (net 2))
 (segment (start 61.655 53.745) (end 63.8 53.745) (width 0.2) (layer "B.Cu") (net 2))
 (segment (start 63.8 53.745) (end 92.342 53.745) (width 0.2) (layer "B.Cu") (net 2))
 (segment (start 30.141 53.745) (end 58.005 53.745) (width 0.2) (layer "B.Cu") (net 2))
 (segment (start 34.811 28.171) (end 34.811 27.733) (width 0.2) (layer "B.Cu") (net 2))
 (segment (start 68.55 43.2) (end 68.55 42.6) (width 0.2) (layer "B.Cu") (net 2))
 (segment (start 59.83 51.92) (end 61.605 53.695) (width 0.2) (layer "B.Cu") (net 2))
 (segment (start 82.743 37.657) (end 81.175 39.225) (width 0.2) (layer "B.Cu") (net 2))
 (segment (start 35.643 27.733) (end 34.811 27.733) (width 0.2) (layer "B.Cu") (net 2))
 (segment (start 61.605 53.695) (end 61.655 53.745) (width 0.2) (layer "B.Cu") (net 2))
 (segment (start 59.83 51.92) (end 68.55 43.2) (width 0.2) (layer "B.Cu") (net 2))
 (segment (start 68.55 42.6) (end 68.55 31.416) (width 0.2) (layer "B.Cu") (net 2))
 (segment (start 46.4085 50.5915) (end 45.8 49.983) (width 0.2) (layer "B.Cu") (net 2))
 (segment (start 15.254 38.858) (end 30.141 53.745) (width 0.2) (layer "B.Cu") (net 2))
 (segment (start 59.83 51.92) (end 47.737 51.92) (width 0.2) (layer "B.Cu") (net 2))
 (segment (start 82.743 27.384) (end 82.743 37.657) (width 0.2) (layer "B.Cu") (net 2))
 (segment (start 34.43 55.73) (end 31.294 52.594) (width 0.2) (layer "F.Cu") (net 10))
 (segment (start 31.294 38.35) (end 31.294 52) (width 0.2) (layer "F.Cu") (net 10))
 (segment (start 39.811 29.833) (end 31.294 38.35) (width 0.2) (layer "F.Cu") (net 10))
 (segment (start 31.294 52.594) (end 31.294 52) (width 0.2) (layer "F.Cu") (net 10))
 (segment (start 57.29 55.73) (end 57.29 50.083) (width 0.2) (layer "F.Cu") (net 7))
 (segment (start 57.29 50.083) (end 60.947 46.426) (width 0.2) (layer "F.Cu") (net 7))
 (segment (start 18.276701 73.39467) (end 23.932031 79.05) (width 0.2) (layer "F.Cu") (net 3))
 (segment (start 18.276701 59.053759) (end 18.276701 73.39467) (width 0.2) (layer "F.Cu") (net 3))
 (segment (start 10.25 6.3) (end 12.15 8.2) (width 0.2) (layer "F.Cu") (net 3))
 (segment (start 41.59 79.05) (end 44.59 76.05) (width 0.2) (layer "F.Cu") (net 3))
 (segment (start 12.15 8.2) (end 12.15 52.927058) (width 0.2) (layer "F.Cu") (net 3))
 (segment (start 12.15 52.927058) (end 18.276701 59.053759) (width 0.2) (layer "F.Cu") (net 3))
 (segment (start 23.932031 79.05) (end 41.59 79.05) (width 0.2) (layer "F.Cu") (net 3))
 (segment (start 17.015686 58.27) (end 12.15 53.404314) (width 0.2) (layer "B.Cu") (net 6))
 (segment (start 21.73 58.27) (end 17.015686 58.27) (width 0.2) (layer "B.Cu") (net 6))
 (segment (start 12.15 5.1) (end 10.25 3.2) (width 0.2) (layer "B.Cu") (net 6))
 (segment (start 12.15 53.404314) (end 12.15 5.1) (width 0.2) (layer "B.Cu") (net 6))
 (segment (start 78.6135 54.7265) (end 78.6135 38.6135) (width 0.2) (layer "F.Cu") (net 14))
 (segment (start 78.6135 38.6135) (end 87.743 29.484) (width 0.2) (layer "F.Cu") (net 14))
 (segment (start 77.61 55.73) (end 78.6135 54.7265) (width 0.2) (layer "F.Cu") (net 14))
 (segment (start 11.75 17.5) (end 5.75 11.5) (width 0.2) (layer "B.Cu") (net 5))
 (segment (start 11.75 53.57) (end 11.75 17.5) (width 0.2) (layer "B.Cu") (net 5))
 (segment (start 21.73 73.51) (end 19.075 70.855) (width 0.2) (layer "B.Cu") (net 5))
 (segment (start 16 79.24) (end 21.73 73.51) (width 0.2) (layer "B.Cu") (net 5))
 (segment (start 19.075 70.855) (end 19.075 60.895) (width 0.2) (layer "B.Cu") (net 5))
 (segment (start 16 90.3) (end 16 79.24) (width 0.2) (layer "B.Cu") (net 5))
 (segment (start 19.075 60.895) (end 11.75 53.57) (width 0.2) (layer "B.Cu") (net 5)))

